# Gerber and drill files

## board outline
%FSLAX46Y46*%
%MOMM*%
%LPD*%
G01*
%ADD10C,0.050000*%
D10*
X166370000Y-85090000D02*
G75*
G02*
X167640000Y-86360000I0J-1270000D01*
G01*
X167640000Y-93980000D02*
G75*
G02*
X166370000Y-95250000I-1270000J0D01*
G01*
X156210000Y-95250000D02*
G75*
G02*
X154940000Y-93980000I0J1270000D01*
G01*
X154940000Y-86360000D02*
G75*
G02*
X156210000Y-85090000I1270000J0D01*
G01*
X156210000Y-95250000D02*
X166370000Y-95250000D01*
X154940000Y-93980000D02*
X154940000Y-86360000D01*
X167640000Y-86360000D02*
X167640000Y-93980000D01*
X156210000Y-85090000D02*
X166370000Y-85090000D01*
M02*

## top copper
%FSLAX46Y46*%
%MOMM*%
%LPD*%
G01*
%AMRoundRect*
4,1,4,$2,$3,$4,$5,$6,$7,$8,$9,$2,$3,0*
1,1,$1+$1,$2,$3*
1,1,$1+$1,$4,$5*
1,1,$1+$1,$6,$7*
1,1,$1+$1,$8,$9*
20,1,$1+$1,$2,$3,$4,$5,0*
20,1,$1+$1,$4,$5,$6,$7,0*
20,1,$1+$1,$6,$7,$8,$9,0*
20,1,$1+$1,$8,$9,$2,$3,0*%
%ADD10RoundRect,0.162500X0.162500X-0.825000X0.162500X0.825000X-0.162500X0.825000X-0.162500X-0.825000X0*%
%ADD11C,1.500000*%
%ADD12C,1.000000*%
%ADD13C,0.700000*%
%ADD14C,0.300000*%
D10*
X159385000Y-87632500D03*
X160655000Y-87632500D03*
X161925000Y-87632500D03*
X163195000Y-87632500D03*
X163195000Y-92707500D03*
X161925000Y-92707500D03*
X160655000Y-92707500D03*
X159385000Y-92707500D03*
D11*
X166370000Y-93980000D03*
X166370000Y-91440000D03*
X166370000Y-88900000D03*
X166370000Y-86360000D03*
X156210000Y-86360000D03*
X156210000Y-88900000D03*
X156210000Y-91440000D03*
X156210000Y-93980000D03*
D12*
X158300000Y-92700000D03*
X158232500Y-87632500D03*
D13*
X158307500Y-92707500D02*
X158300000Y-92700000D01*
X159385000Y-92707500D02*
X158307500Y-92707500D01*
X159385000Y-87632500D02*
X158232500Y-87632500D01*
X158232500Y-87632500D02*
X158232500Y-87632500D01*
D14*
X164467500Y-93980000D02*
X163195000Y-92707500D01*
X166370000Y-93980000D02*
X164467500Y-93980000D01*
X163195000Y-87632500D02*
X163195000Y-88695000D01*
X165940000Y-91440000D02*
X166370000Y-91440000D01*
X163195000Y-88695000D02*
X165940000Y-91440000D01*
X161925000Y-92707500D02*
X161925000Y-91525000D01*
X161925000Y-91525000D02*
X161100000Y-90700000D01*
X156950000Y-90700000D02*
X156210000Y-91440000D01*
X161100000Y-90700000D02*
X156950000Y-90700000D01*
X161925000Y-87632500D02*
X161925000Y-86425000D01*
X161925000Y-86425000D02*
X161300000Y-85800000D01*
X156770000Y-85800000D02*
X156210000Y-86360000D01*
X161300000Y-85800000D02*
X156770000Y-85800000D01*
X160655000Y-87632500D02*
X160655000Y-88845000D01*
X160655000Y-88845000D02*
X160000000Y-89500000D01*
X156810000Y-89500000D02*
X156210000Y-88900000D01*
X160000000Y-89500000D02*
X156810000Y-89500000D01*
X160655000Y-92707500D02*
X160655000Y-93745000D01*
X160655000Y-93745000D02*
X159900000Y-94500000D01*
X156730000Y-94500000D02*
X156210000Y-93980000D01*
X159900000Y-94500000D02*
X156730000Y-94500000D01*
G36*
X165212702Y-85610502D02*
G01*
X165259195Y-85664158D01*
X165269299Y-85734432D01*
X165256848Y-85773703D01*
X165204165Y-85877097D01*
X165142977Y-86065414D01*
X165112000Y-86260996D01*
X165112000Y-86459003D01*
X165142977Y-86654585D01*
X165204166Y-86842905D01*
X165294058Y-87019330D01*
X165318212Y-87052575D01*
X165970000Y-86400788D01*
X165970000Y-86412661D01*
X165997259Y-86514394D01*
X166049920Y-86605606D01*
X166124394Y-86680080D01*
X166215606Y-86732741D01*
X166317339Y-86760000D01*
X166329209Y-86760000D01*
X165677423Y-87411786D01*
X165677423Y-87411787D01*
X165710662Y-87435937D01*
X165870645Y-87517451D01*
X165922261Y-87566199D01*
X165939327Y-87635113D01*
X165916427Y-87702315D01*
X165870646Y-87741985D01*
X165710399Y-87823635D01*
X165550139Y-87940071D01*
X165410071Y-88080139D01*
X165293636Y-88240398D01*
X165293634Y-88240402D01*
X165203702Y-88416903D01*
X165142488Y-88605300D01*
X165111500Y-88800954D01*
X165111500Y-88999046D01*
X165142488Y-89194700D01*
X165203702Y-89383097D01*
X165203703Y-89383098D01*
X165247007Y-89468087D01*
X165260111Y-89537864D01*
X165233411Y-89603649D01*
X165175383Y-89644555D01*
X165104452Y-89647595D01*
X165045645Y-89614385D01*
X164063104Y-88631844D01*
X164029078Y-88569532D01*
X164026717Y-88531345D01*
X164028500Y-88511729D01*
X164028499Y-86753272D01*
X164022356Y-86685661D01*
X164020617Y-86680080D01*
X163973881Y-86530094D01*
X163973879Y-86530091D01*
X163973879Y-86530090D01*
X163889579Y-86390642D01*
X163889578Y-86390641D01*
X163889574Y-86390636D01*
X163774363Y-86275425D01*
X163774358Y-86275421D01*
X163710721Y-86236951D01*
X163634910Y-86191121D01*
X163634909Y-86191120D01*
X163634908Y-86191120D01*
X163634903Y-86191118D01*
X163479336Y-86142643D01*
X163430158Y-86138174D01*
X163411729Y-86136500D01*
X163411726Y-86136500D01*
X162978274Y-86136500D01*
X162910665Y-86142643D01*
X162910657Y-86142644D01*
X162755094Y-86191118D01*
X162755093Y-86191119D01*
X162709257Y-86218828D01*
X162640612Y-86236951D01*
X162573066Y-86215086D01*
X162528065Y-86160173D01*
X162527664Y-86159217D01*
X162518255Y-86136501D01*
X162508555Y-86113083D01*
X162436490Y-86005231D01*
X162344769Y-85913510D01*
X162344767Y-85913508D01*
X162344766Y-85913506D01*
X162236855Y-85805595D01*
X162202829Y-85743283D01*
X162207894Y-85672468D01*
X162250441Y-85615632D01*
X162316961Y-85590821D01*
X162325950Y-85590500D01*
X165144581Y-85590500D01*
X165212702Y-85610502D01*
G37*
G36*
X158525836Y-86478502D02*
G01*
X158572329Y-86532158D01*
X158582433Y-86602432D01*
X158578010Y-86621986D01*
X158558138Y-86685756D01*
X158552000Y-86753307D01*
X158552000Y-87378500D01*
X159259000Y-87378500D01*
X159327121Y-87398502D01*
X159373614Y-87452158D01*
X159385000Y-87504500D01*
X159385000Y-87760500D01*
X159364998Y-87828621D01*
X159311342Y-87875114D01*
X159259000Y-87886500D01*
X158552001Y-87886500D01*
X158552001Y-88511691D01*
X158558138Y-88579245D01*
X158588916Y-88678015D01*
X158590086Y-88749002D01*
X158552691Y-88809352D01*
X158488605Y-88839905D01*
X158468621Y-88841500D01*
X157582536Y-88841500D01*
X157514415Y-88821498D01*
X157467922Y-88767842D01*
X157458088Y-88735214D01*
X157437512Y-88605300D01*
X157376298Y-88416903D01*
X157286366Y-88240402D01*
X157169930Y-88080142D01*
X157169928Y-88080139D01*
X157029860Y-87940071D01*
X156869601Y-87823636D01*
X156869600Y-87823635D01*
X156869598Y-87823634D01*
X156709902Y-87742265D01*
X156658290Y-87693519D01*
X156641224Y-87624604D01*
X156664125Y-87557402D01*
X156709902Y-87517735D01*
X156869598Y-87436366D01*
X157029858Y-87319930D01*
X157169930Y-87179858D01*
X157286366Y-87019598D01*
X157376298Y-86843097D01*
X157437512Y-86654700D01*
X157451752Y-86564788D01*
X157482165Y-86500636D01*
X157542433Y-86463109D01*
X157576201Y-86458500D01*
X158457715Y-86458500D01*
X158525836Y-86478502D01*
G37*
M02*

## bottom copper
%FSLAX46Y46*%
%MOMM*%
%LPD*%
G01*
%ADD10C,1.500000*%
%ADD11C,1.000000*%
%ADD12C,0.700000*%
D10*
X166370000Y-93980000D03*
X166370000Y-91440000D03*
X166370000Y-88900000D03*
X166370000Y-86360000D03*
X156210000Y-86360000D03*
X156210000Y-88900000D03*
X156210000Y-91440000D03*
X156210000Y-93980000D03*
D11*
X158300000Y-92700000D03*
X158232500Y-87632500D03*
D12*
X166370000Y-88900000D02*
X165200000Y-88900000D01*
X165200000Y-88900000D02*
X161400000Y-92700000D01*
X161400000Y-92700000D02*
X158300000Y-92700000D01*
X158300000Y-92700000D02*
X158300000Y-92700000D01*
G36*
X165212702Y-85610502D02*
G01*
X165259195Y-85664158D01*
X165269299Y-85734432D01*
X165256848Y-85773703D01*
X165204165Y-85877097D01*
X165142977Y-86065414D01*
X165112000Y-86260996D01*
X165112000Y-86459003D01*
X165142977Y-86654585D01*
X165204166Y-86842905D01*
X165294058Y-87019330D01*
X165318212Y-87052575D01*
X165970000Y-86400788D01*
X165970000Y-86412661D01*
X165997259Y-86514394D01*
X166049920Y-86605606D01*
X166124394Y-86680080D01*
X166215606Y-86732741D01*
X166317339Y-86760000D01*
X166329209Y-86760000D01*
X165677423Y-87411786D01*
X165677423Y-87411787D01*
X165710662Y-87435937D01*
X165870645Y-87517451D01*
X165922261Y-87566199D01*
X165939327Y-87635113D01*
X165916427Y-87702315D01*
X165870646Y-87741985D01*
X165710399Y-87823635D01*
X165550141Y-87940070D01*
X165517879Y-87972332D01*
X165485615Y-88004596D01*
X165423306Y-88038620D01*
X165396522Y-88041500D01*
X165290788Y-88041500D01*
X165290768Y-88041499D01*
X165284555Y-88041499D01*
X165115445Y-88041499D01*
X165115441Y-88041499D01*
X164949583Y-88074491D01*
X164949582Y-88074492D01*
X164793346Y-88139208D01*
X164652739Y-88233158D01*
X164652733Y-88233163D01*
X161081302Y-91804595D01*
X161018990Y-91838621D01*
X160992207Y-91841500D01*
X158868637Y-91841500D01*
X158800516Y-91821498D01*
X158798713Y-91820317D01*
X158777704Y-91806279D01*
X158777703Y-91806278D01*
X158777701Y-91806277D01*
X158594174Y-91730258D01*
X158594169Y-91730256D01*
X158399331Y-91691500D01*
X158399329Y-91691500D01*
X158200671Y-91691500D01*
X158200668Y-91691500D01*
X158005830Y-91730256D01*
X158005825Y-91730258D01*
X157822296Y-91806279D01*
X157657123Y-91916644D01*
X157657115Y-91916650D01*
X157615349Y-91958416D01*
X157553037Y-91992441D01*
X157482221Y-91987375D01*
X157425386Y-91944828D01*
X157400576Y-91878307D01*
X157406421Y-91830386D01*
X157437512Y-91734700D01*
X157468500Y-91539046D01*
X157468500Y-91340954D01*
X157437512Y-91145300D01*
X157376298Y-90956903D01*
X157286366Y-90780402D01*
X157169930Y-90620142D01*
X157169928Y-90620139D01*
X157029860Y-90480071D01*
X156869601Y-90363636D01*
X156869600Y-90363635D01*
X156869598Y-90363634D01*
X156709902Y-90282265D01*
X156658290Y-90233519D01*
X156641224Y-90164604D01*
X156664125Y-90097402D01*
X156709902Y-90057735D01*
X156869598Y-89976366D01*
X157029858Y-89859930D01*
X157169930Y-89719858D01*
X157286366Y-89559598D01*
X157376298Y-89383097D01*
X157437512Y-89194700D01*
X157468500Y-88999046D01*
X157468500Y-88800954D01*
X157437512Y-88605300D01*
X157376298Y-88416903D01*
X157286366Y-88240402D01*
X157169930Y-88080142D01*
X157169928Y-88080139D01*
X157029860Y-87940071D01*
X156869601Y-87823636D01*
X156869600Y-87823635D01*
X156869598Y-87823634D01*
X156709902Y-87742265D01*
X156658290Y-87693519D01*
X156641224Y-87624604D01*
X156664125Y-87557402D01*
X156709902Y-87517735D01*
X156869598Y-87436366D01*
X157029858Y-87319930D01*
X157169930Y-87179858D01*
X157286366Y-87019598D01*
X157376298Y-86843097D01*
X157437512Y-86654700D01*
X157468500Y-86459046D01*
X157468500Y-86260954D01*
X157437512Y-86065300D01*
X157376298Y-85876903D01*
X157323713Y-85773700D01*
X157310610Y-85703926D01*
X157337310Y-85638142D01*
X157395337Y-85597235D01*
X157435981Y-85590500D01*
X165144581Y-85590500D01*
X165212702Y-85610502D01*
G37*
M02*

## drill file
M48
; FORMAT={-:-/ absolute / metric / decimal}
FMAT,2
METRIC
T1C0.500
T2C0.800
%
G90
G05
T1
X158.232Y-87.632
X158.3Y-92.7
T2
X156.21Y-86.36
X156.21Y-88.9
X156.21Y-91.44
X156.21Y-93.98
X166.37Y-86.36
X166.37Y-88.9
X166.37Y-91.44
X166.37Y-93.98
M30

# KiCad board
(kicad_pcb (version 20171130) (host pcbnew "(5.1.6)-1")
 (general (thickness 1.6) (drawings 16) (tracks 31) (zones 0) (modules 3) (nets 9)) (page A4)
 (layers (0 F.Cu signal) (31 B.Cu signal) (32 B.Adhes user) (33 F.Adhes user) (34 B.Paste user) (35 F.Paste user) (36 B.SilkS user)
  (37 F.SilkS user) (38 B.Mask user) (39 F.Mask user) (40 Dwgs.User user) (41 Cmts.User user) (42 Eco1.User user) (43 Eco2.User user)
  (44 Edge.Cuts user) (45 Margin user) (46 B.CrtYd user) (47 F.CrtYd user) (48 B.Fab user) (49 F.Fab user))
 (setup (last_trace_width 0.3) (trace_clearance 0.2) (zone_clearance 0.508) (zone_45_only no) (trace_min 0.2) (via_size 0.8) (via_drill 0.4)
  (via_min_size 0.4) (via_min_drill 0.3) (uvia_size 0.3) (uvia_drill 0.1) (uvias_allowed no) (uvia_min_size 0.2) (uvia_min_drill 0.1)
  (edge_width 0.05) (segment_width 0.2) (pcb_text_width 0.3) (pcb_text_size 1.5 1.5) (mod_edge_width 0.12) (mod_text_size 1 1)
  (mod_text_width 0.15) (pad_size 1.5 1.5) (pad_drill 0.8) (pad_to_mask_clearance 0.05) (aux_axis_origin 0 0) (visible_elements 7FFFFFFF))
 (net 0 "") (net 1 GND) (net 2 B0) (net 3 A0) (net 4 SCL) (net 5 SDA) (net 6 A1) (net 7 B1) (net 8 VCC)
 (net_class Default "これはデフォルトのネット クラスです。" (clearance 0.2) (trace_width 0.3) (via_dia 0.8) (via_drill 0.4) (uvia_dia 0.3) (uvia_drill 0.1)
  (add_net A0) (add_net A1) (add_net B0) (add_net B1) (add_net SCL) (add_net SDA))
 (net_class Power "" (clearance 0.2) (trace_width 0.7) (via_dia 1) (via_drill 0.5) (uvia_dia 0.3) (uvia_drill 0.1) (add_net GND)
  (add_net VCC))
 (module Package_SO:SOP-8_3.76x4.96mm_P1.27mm (layer F.Cu) (at 161.29 90.17 90)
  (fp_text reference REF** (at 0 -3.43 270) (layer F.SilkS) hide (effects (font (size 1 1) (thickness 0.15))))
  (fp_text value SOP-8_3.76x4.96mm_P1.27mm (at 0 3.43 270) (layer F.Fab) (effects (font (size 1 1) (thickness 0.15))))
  (pad 8 smd roundrect (at 2.5375 -1.905 90) (size 1.975 0.65) (layers F.Cu F.Paste F.Mask) (roundrect_rratio 0.25) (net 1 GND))
  (pad 7 smd roundrect (at 2.5375 -0.635 90) (size 1.975 0.65) (layers F.Cu F.Paste F.Mask) (roundrect_rratio 0.25) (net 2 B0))
  (pad 6 smd roundrect (at 2.5375 0.635 90) (size 1.975 0.65) (layers F.Cu F.Paste F.Mask) (roundrect_rratio 0.25) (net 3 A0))
  (pad 5 smd roundrect (at 2.5375 1.905 90) (size 1.975 0.65) (layers F.Cu F.Paste F.Mask) (roundrect_rratio 0.25) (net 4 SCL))
  (pad 4 smd roundrect (at -2.5375 1.905 90) (size 1.975 0.65) (layers F.Cu F.Paste F.Mask) (roundrect_rratio 0.25) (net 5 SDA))
  (pad 3 smd roundrect (at -2.5375 0.635 90) (size 1.975 0.65) (layers F.Cu F.Paste F.Mask) (roundrect_rratio 0.25) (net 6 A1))
  (pad 2 smd roundrect (at -2.5375 -0.635 90) (size 1.975 0.65) (layers F.Cu F.Paste F.Mask) (roundrect_rratio 0.25) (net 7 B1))
  (pad 1 smd roundrect (at -2.5375 -1.905 90) (size 1.975 0.65) (layers F.Cu F.Paste F.Mask) (roundrect_rratio 0.25) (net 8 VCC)))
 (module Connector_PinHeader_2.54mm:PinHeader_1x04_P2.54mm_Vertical (layer F.Cu) (at 166.37 90.17 90)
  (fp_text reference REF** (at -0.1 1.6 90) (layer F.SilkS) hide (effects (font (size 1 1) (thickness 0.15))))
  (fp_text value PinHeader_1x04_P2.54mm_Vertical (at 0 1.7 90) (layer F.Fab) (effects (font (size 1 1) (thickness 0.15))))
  (pad 1 thru_hole circle (at -3.81 0 90) (size 1.5 1.5) (drill 0.8) (layers *.Cu *.Mask) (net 5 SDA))
  (pad 2 thru_hole circle (at -1.27 0 90) (size 1.5 1.5) (drill 0.8) (layers *.Cu *.Mask) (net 4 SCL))
  (pad 3 thru_hole circle (at 1.27 0 90) (size 1.5 1.5) (drill 0.8) (layers *.Cu *.Mask) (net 8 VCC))
  (pad 4 thru_hole circle (at 3.81 0 90) (size 1.5 1.5) (drill 0.8) (layers *.Cu *.Mask) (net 1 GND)))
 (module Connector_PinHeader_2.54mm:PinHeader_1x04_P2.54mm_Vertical (layer F.Cu) (at 156.21 90.17 90)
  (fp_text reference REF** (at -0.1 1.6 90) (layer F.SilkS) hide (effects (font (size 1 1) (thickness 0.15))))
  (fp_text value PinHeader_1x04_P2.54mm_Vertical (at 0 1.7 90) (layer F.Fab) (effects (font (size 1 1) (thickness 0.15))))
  (pad 4 thru_hole circle (at 3.81 0 90) (size 1.5 1.5) (drill 0.8) (layers *.Cu *.Mask) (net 3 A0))
  (pad 3 thru_hole circle (at 1.27 0 90) (size 1.5 1.5) (drill 0.8) (layers *.Cu *.Mask) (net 2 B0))
  (pad 2 thru_hole circle (at -1.27 0 90) (size 1.5 1.5) (drill 0.8) (layers *.Cu *.Mask) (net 6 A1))
  (pad 1 thru_hole circle (at -3.81 0 90) (size 1.5 1.5) (drill 0.8) (layers *.Cu *.Mask) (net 7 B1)))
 (gr_arc (start 166.37 86.36) (end 167.64 86.36) (angle -90) (layer Edge.Cuts) (width 0.05))
 (gr_arc (start 166.37 93.98) (end 166.37 95.25) (angle -90) (layer Edge.Cuts) (width 0.05))
 (gr_arc (start 156.21 93.98) (end 154.94 93.98) (angle -90) (layer Edge.Cuts) (width 0.05))
 (gr_arc (start 156.21 86.36) (end 156.21 85.09) (angle -90) (layer Edge.Cuts) (width 0.05))
 (gr_line (start 156.21 95.25) (end 166.37 95.25) (layer Edge.Cuts) (width 0.05))
 (gr_line (start 154.94 93.98) (end 154.94 86.36) (layer Edge.Cuts) (width 0.05))
 (gr_line (start 167.64 86.36) (end 167.64 93.98) (layer Edge.Cuts) (width 0.05))
 (gr_line (start 156.21 85.09) (end 166.37 85.09) (layer Edge.Cuts) (width 0.05))
 (segment (start 166.37 88.9) (end 165.2 88.9) (width 0.7) (layer B.Cu) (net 8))
 (segment (start 165.2 88.9) (end 161.4 92.7) (width 0.7) (layer B.Cu) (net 8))
 (segment (start 161.4 92.7) (end 158.3 92.7) (width 0.7) (layer B.Cu) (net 8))
 (segment (start 158.3 92.7) (end 158.3 92.7) (width 0.7) (layer B.Cu) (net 8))
 (via (at 158.3 92.7) (size 1) (drill 0.5) (layers F.Cu B.Cu) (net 8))
 (segment (start 158.3075 92.7075) (end 158.3 92.7) (width 0.7) (layer F.Cu) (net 8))
 (segment (start 159.385 92.7075) (end 158.3075 92.7075) (width 0.7) (layer F.Cu) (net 8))
 (segment (start 159.385 87.6325) (end 158.2325 87.6325) (width 0.7) (layer F.Cu) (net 1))
 (segment (start 158.2325 87.6325) (end 158.2325 87.6325) (width 0.7) (layer F.Cu) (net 1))
 (via (at 158.2325 87.6325) (size 1) (drill 0.5) (layers F.Cu B.Cu) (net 1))
 (segment (start 164.4675 93.98) (end 163.195 92.7075) (width 0.3) (layer F.Cu) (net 5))
 (segment (start 166.37 93.98) (end 164.4675 93.98) (width 0.3) (layer F.Cu) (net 5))
 (segment (start 163.195 87.6325) (end 163.195 88.695) (width 0.3) (layer F.Cu) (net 4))
 (segment (start 165.94 91.44) (end 166.37 91.44) (width 0.3) (layer F.Cu) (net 4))
 (segment (start 163.195 88.695) (end 165.94 91.44) (width 0.3) (layer F.Cu) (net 4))
 (segment (start 161.925 92.7075) (end 161.925 91.525) (width 0.3) (layer F.Cu) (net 6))
 (segment (start 161.925 91.525) (end 161.1 90.7) (width 0.3) (layer F.Cu) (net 6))
 (segment (start 156.95 90.7) (end 156.21 91.44) (width 0.3) (layer F.Cu) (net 6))
 (segment (start 161.1 90.7) (end 156.95 90.7) (width 0.3) (layer F.Cu) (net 6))
 (segment (start 161.925 87.6325) (end 161.925 86.425) (width 0.3) (layer F.Cu) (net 3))
 (segment (start 161.925 86.425) (end 161.3 85.8) (width 0.3) (layer F.Cu) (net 3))
 (segment (start 156.77 85.8) (end 156.21 86.36) (width 0.3) (layer F.Cu) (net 3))
 (segment (start 161.3 85.8) (end 156.77 85.8) (width 0.3) (layer F.Cu) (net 3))
 (segment (start 160.655 87.6325) (end 160.655 88.845) (width 0.3) (layer F.Cu) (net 2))
 (segment (start 160.655 88.845) (end 160 89.5) (width 0.3) (layer F.Cu) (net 2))
 (segment (start 156.81 89.5) (end 156.21 88.9) (width 0.3) (layer F.Cu) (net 2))
 (segment (start 160 89.5) (end 156.81 89.5) (width 0.3) (layer F.Cu) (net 2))
 (segment (start 160.655 92.7075) (end 160.655 93.745) (width 0.3) (layer F.Cu) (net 7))
 (segment (start 160.655 93.745) (end 159.9 94.5) (width 0.3) (layer F.Cu) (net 7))
 (segment (start 156.73 94.5) (end 156.21 93.98) (width 0.3) (layer F.Cu) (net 7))
 (segment (start 159.9 94.5) (end 156.73 94.5) (width 0.3) (layer F.Cu) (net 7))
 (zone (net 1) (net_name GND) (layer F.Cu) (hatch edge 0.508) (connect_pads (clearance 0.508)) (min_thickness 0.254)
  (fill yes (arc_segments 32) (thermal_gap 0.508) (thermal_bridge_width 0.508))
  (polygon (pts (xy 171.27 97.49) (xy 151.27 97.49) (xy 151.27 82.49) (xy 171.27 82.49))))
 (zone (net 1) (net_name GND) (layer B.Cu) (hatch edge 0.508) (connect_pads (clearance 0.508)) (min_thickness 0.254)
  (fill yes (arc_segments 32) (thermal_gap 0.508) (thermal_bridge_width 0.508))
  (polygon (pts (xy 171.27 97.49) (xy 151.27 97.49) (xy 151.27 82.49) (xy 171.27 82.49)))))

